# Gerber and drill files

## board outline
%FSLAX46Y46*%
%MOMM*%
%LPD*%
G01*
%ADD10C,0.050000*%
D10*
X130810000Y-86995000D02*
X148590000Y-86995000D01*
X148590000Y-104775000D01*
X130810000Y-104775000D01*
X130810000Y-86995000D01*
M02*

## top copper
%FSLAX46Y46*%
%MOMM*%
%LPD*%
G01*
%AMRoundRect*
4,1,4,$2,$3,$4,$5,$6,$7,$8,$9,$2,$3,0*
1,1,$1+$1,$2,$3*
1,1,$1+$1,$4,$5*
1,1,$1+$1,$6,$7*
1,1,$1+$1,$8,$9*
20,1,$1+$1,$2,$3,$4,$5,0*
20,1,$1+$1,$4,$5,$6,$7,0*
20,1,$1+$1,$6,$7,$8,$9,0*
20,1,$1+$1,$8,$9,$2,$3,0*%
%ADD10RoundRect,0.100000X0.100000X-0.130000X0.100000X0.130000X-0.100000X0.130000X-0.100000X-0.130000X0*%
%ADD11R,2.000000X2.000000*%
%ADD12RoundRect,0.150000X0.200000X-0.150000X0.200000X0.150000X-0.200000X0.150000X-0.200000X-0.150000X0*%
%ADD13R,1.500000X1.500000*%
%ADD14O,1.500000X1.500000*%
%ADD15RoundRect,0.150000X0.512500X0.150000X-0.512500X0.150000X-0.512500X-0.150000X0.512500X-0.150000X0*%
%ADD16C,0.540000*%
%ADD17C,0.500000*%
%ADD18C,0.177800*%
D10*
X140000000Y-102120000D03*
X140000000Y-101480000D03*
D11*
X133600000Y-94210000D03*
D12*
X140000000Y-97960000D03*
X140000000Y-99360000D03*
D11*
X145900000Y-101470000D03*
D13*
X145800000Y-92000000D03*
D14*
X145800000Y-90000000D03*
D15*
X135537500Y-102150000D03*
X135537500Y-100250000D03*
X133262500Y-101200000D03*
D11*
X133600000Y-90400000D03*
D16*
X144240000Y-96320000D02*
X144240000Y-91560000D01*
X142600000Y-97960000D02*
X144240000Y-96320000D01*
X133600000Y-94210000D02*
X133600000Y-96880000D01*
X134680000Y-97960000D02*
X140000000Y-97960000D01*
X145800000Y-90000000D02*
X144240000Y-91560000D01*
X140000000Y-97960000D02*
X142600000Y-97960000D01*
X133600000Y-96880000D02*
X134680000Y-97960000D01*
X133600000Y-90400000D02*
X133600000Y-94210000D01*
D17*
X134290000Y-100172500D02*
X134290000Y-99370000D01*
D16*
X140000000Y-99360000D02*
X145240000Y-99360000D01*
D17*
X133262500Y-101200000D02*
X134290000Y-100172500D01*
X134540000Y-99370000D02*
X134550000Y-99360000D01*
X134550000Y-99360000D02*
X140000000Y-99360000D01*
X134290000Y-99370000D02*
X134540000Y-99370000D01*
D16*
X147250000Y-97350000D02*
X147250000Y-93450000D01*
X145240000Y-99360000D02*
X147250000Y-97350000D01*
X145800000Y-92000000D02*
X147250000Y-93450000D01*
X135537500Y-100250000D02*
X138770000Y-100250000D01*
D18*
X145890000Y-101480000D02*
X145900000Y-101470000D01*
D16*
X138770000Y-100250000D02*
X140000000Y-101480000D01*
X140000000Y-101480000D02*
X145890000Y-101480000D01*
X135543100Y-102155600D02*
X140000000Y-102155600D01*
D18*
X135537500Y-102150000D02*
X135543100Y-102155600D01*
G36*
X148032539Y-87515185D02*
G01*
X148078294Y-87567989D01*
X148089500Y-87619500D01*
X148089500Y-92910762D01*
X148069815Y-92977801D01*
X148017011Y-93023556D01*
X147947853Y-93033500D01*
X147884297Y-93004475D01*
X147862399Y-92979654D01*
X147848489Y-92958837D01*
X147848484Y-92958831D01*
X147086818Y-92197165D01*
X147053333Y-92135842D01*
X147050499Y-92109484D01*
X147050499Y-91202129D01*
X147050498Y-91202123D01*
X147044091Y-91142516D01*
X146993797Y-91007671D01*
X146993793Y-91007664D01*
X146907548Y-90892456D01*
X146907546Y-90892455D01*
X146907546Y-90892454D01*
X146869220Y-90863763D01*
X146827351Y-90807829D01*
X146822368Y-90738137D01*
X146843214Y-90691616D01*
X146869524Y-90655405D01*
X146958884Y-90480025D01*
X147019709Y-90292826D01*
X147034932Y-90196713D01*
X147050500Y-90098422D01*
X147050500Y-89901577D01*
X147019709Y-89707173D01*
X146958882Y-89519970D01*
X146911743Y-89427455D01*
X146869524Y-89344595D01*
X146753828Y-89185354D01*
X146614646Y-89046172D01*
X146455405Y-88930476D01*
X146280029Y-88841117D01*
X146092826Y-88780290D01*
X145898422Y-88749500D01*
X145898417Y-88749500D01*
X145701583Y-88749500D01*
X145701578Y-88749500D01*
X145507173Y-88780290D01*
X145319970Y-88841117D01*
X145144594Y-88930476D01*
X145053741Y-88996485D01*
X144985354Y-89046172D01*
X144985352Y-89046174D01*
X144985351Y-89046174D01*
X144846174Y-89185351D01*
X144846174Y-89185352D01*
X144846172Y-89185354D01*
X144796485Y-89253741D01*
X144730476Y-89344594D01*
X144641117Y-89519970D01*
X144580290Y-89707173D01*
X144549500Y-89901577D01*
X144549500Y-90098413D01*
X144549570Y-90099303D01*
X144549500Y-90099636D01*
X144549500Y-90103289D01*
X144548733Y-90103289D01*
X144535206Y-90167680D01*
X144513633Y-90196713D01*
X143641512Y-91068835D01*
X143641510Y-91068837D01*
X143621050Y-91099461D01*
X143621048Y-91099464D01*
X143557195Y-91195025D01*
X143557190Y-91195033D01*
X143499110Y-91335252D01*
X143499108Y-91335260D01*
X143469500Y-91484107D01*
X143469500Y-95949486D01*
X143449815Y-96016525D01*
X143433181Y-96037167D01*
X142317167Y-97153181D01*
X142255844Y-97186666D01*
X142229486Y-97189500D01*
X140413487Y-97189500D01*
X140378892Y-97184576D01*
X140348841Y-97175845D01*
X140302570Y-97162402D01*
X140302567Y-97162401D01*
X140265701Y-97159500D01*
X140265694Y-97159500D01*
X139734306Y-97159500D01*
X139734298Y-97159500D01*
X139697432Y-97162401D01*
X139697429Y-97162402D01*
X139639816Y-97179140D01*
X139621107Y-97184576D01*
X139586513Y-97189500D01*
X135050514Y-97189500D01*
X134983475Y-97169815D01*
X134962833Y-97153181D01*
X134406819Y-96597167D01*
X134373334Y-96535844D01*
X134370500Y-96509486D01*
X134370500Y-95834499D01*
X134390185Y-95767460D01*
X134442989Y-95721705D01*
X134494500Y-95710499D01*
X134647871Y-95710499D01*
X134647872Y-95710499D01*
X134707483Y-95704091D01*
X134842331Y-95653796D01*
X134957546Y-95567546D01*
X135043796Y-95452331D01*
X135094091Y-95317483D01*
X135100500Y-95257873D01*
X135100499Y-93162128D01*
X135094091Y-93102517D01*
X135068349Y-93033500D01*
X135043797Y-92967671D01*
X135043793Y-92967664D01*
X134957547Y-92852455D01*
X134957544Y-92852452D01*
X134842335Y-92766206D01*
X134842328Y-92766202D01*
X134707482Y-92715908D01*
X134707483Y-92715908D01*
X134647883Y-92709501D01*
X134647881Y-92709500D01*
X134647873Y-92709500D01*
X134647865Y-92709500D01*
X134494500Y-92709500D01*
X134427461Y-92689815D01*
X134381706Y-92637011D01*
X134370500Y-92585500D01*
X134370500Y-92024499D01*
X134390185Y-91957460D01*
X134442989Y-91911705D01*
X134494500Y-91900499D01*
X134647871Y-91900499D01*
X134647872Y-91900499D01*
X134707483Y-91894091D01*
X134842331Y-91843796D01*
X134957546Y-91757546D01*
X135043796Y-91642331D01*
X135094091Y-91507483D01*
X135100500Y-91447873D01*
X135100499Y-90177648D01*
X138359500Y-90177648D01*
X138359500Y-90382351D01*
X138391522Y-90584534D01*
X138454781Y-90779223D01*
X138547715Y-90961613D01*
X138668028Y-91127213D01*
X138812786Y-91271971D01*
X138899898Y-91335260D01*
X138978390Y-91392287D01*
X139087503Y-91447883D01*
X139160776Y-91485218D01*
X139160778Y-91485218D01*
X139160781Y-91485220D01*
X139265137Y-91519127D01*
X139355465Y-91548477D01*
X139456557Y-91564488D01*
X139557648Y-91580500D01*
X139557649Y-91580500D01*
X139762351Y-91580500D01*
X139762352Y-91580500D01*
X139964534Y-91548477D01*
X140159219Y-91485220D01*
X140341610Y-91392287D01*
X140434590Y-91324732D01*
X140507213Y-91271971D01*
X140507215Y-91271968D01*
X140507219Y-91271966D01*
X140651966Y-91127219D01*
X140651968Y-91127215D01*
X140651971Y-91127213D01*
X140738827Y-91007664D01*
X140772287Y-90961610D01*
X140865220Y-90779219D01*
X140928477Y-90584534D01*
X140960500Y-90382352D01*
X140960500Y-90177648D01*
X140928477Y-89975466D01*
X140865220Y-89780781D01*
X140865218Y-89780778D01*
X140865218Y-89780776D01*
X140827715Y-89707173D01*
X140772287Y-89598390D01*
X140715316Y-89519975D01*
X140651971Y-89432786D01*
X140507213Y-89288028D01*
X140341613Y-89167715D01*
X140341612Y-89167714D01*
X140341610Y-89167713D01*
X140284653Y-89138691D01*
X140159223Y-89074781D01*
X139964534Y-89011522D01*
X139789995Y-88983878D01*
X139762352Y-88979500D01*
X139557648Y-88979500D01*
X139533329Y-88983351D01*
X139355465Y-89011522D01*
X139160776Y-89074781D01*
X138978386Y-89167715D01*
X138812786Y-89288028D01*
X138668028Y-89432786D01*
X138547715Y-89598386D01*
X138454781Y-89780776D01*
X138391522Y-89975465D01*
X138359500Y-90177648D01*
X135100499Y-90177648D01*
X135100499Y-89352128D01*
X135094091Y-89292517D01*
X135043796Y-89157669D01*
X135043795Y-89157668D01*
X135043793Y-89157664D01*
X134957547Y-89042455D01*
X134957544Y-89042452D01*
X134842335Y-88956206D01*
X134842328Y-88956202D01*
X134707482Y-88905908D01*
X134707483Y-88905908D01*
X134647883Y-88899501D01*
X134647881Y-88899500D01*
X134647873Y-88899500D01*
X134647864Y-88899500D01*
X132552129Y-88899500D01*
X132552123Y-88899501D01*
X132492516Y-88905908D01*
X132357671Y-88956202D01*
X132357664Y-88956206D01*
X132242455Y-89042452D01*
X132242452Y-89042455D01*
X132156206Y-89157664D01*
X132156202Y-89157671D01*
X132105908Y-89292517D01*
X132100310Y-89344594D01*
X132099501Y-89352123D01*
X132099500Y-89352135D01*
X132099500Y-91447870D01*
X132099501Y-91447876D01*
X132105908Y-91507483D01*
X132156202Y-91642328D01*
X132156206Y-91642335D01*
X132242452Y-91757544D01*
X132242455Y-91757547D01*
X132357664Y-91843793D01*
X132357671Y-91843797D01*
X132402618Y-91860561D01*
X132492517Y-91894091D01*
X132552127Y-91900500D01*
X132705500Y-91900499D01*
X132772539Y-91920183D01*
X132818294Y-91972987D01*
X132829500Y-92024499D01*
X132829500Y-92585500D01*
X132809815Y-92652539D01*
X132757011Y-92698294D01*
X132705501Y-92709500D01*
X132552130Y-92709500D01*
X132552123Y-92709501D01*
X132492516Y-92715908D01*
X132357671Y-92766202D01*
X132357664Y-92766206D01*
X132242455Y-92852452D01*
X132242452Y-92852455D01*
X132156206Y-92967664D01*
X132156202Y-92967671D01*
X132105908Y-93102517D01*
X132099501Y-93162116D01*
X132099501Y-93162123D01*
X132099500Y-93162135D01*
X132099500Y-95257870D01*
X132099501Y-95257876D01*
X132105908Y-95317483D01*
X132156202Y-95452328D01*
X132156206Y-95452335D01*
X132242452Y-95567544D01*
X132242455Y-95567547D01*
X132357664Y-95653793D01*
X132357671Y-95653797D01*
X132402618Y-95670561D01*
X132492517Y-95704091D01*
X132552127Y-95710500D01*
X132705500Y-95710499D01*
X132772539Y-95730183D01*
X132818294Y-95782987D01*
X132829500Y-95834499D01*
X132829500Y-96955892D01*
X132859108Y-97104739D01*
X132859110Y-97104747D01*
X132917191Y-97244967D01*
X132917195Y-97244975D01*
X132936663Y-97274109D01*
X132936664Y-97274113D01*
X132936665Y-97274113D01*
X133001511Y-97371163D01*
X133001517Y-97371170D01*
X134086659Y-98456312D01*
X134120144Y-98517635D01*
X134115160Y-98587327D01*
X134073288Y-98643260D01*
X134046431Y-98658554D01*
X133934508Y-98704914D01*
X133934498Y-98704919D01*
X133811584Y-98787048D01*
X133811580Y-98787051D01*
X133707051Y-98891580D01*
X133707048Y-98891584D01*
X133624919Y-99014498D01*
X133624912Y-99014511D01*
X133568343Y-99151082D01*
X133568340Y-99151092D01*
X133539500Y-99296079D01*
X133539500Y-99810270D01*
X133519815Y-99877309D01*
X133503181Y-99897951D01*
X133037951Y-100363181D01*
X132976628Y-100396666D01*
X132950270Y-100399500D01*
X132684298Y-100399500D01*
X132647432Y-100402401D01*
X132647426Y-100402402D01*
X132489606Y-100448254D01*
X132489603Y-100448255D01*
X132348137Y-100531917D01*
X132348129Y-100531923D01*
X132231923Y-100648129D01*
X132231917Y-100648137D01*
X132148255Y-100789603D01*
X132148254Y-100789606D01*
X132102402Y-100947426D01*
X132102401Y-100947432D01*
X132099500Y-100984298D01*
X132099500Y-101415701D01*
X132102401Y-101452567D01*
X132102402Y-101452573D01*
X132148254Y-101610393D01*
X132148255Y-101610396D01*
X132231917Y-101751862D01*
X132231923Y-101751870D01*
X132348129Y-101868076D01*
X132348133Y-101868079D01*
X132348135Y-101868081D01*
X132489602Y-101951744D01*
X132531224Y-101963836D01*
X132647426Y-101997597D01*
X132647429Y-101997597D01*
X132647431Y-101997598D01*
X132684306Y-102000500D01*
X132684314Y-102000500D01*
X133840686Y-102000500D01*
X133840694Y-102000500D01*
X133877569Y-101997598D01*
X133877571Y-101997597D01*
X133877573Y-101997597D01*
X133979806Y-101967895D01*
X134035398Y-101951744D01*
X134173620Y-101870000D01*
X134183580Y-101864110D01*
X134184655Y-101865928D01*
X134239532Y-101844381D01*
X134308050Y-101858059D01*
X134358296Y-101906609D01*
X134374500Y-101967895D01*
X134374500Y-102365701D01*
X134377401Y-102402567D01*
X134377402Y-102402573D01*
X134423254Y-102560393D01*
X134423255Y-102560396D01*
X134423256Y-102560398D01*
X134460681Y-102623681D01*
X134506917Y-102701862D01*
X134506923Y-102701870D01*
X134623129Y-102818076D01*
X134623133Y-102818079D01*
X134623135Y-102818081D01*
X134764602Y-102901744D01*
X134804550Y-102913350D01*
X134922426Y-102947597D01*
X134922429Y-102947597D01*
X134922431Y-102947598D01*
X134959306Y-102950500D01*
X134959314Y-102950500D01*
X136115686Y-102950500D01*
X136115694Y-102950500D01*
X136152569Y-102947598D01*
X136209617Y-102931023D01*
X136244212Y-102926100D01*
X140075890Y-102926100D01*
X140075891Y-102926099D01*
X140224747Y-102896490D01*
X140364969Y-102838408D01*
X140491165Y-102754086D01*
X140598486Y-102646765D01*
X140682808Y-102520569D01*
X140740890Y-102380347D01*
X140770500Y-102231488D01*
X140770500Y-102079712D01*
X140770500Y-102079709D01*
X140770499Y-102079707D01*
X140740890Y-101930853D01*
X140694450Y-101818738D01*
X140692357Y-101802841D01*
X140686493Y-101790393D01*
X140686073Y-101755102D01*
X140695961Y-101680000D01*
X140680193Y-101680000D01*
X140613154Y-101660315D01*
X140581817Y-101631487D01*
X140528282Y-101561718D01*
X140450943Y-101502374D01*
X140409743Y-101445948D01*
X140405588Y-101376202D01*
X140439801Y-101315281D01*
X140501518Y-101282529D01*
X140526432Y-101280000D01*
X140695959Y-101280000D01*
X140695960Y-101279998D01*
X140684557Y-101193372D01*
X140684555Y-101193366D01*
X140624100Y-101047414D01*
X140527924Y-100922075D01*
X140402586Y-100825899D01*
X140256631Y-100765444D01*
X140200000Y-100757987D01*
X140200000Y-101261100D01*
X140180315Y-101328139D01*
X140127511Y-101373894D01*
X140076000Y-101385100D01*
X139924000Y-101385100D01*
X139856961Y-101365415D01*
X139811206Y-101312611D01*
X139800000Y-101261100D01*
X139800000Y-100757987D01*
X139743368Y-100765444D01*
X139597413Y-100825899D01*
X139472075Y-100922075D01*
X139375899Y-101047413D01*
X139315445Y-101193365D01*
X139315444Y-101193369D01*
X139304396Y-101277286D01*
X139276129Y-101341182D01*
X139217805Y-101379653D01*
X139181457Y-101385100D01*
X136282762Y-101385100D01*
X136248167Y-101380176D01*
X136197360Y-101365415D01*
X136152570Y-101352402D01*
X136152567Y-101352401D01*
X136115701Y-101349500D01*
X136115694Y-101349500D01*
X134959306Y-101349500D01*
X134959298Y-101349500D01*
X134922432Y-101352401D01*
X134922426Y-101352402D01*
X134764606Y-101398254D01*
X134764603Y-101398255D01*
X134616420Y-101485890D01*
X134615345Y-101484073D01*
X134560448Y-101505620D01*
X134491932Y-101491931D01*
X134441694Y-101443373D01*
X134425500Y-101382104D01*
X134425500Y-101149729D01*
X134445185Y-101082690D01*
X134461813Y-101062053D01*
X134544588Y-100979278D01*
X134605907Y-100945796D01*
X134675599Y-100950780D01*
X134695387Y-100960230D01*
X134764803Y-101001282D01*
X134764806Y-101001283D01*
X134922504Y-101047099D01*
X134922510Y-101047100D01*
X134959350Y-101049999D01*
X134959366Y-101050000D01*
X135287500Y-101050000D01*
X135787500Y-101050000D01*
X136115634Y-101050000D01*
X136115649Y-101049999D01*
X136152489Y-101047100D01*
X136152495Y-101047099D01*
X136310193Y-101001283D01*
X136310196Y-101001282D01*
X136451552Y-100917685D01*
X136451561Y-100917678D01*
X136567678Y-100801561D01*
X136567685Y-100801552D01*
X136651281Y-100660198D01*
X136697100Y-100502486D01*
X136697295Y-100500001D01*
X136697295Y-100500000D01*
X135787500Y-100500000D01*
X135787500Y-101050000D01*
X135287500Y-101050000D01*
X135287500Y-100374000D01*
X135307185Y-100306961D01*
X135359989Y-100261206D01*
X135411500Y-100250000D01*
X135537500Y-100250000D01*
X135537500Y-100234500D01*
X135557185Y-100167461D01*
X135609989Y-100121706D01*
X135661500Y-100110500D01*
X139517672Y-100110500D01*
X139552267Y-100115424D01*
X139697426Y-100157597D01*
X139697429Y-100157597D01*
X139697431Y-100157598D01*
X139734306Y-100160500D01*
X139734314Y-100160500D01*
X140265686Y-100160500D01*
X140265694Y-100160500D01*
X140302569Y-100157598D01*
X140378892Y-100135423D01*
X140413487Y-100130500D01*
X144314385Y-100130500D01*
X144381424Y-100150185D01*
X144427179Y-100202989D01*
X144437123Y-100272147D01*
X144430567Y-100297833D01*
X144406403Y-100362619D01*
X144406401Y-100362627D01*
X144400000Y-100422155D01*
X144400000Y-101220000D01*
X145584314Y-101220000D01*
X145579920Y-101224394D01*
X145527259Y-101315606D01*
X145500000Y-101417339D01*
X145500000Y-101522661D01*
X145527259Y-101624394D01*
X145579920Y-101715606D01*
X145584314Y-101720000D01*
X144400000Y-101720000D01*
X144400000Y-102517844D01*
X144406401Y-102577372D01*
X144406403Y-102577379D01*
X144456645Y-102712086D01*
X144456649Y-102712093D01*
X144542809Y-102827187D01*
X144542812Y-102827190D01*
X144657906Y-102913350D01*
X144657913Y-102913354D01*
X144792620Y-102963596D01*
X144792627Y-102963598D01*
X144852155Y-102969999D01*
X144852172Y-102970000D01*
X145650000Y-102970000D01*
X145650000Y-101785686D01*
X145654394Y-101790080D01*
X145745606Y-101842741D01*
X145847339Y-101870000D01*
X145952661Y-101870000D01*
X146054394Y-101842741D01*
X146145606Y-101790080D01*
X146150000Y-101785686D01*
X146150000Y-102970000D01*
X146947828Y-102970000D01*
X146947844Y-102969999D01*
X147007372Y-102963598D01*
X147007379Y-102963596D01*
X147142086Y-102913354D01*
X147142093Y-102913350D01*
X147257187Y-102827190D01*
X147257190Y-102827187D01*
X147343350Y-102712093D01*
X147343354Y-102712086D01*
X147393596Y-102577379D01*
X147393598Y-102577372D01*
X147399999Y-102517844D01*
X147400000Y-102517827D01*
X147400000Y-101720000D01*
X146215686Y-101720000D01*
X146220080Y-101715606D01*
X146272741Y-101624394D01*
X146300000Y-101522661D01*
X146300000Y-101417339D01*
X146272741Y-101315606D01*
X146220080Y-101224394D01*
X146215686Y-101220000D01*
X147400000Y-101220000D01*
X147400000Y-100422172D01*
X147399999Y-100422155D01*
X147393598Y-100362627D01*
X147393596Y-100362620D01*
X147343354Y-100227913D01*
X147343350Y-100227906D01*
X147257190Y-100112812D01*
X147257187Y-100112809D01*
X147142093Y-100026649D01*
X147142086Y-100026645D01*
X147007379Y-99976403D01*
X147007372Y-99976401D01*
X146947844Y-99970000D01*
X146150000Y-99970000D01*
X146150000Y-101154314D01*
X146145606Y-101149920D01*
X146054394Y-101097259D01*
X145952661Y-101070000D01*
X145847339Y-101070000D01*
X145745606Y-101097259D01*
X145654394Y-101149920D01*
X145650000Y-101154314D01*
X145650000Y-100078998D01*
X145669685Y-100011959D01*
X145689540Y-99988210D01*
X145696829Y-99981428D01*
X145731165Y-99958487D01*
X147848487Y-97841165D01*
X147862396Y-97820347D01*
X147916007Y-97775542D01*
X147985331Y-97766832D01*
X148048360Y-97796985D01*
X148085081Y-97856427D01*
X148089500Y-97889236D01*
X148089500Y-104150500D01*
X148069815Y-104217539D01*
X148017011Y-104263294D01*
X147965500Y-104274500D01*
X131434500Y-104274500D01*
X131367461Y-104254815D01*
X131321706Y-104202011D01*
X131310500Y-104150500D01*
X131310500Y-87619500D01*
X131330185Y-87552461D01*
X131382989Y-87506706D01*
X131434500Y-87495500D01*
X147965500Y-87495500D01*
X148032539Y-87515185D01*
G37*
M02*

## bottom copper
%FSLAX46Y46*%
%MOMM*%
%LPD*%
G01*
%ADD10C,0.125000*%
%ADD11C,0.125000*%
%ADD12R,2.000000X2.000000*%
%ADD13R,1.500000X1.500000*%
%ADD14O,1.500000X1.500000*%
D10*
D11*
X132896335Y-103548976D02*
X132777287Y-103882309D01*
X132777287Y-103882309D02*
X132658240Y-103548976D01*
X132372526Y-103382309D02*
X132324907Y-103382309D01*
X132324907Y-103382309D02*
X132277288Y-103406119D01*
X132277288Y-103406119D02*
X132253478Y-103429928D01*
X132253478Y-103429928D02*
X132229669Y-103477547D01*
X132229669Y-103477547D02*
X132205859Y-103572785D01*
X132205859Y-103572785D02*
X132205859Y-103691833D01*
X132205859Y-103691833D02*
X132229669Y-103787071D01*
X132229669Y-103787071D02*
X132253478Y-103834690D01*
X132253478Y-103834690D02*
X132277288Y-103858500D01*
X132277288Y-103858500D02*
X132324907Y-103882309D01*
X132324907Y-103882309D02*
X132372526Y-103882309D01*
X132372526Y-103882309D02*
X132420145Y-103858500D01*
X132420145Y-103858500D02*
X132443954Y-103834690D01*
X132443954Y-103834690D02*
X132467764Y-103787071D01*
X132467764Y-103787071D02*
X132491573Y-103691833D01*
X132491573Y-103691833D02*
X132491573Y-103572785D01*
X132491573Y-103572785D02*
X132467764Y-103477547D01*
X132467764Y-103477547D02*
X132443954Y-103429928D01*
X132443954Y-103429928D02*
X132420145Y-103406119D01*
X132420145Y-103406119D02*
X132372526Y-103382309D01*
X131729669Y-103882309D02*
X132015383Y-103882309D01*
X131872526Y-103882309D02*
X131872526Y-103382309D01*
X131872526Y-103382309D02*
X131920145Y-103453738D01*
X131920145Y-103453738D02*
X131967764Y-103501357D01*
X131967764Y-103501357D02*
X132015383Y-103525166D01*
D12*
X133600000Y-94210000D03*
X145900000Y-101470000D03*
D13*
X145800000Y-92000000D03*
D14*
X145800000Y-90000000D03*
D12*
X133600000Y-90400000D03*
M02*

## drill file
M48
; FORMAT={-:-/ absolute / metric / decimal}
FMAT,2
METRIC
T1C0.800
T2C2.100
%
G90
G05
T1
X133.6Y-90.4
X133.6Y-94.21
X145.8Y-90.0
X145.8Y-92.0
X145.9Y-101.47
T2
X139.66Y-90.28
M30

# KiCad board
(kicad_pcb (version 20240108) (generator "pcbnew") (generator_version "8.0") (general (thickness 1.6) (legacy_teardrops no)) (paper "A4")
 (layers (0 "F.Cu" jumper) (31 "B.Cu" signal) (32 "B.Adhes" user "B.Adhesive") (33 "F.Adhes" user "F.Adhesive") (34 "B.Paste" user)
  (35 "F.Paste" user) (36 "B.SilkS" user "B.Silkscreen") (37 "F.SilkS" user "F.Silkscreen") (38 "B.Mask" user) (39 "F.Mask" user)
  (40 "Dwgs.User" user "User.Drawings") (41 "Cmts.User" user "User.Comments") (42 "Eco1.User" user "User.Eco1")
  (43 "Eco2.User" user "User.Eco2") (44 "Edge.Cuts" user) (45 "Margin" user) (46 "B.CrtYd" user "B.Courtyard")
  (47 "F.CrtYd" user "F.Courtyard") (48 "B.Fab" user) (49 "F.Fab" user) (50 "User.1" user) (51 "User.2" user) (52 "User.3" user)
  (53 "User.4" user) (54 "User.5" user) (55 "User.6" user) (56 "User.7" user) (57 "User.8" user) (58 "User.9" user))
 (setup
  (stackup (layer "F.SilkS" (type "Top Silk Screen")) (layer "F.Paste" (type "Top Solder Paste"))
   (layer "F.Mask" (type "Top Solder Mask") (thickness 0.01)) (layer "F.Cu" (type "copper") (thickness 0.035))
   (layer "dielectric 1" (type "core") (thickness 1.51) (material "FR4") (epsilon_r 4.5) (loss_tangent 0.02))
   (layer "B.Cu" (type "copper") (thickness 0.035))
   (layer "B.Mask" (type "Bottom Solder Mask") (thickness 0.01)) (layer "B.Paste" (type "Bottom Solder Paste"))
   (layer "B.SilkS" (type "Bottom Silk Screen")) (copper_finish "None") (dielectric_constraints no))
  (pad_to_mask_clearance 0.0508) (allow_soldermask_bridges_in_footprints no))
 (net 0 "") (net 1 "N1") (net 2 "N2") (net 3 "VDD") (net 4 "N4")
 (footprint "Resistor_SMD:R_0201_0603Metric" (layer "F.Cu") (at 140 101.8 90)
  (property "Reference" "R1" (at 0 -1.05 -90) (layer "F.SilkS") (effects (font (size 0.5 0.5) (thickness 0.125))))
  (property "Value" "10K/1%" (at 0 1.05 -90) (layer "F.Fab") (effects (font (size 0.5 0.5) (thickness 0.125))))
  (pad "" smd roundrect (at -0.345 0 90) (size 0.318 0.36) (layers "F.Paste") (roundrect_rratio 0.25))
  (pad "" smd roundrect (at 0.345 0 90) (size 0.318 0.36) (layers "F.Paste") (roundrect_rratio 0.25))
  (pad "1" smd roundrect (at -0.32 0 90) (size 0.46 0.4) (layers "F.Cu" "F.Mask") (roundrect_rratio 0.25) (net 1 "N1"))
  (pad "2" smd roundrect (at 0.32 0 90) (size 0.46 0.4) (layers "F.Cu" "F.Mask") (roundrect_rratio 0.25) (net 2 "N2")))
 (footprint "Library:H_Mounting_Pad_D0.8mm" (layer "F.Cu") (at 133.6 94.21)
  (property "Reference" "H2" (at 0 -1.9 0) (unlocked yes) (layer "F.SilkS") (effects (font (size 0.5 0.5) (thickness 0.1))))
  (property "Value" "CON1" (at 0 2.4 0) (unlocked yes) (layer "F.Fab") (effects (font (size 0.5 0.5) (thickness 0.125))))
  (pad "1" thru_hole rect (at 0 0) (size 2 2) (drill 0.8) (layers "*.Cu" "*.Mask") (remove_unused_layers no) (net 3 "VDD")))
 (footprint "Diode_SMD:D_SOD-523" (layer "F.Cu") (at 140 98.66 -90)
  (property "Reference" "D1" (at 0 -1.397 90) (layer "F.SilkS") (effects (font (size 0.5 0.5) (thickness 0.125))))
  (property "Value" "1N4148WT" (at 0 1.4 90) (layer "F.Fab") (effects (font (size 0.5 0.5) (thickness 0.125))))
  (pad "1" smd roundrect (at -0.7 0 90) (size 0.6 0.7) (layers "F.Cu" "F.Paste" "F.Mask") (roundrect_rratio 0.25) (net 3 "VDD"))
  (pad "2" smd roundrect (at 0.7 0 90) (size 0.6 0.7) (layers "F.Cu" "F.Paste" "F.Mask") (roundrect_rratio 0.25) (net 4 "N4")))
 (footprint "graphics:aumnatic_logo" (layer "F.Cu") (at 140.95 96)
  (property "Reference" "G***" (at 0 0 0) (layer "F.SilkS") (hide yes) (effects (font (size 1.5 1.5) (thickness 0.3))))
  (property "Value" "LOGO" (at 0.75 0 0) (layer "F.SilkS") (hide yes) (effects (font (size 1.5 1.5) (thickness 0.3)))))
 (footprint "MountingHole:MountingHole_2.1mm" (layer "F.Cu") (at 139.66 90.28)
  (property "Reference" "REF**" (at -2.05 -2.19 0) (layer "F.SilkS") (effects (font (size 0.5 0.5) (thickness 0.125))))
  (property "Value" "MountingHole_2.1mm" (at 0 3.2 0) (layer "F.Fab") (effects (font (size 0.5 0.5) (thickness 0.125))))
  (pad "" np_thru_hole circle (at 0 0) (size 2.1 2.1) (drill 2.1) (layers "*.Cu" "*.Mask")))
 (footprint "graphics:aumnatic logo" (layer "F.Cu") (at 139.6 94.65)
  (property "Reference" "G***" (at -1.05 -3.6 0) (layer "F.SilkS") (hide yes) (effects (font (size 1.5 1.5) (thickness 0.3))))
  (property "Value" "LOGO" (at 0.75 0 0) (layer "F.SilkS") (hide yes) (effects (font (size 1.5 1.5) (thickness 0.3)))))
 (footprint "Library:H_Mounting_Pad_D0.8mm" (layer "F.Cu") (at 145.9 101.47)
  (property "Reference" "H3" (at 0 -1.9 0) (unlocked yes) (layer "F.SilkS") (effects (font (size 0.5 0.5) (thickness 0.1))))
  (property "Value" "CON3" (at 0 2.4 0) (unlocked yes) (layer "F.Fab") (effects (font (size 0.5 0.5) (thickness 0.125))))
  (pad "1" thru_hole rect (at 0 0) (size 2 2) (drill 0.8) (layers "*.Cu" "*.Mask") (remove_unused_layers no) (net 2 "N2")))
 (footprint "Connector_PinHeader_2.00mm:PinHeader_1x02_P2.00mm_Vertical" (layer "F.Cu") (at 145.8 92 180)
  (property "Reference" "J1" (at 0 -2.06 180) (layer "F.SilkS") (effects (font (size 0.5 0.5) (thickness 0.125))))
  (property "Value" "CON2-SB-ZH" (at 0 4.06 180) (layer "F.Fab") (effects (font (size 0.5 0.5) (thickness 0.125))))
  (pad "1" thru_hole rect (at 0 0 180) (size 1.5 1.5) (drill 0.8) (layers "*.Cu" "*.Mask") (remove_unused_layers no) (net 4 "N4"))
  (pad "2" thru_hole oval (at 0 2 180) (size 1.5 1.5) (drill 0.8) (layers "*.Cu" "*.Mask") (remove_unused_layers no) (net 3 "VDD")))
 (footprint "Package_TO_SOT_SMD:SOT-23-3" (layer "F.Cu") (at 134.4 101.2 180)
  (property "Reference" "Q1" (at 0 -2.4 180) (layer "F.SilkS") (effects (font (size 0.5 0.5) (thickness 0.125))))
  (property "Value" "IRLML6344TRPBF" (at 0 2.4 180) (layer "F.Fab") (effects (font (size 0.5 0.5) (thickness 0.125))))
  (pad "1" smd roundrect (at -1.1375 -0.95 180) (size 1.325 0.6) (layers "F.Cu" "F.Paste" "F.Mask") (roundrect_rratio 0.25) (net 1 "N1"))
  (pad "2" smd roundrect (at -1.1375 0.95 180) (size 1.325 0.6) (layers "F.Cu" "F.Paste" "F.Mask") (roundrect_rratio 0.25) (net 2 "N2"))
  (pad "3" smd roundrect (at 1.1375 0 180) (size 1.325 0.6) (layers "F.Cu" "F.Paste" "F.Mask") (roundrect_rratio 0.25) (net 4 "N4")))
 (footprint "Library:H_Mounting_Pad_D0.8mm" (layer "F.Cu") (at 133.6 90.4)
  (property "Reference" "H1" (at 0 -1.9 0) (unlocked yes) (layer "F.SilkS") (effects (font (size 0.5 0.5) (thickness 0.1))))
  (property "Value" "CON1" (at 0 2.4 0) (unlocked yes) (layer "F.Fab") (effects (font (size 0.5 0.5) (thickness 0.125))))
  (pad "1" thru_hole rect (at 0 0) (size 2 2) (drill 0.8) (layers "*.Cu" "*.Mask") (remove_unused_layers no) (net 3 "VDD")))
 (gr_rect (start 130.81 86.995) (end 148.59 104.775) (stroke (width 0.05) (type default)) (fill none) (layer "Edge.Cuts"))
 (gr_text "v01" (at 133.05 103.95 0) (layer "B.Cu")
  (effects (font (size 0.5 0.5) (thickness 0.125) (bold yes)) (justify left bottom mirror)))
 (segment (start 144.24 96.32) (end 144.24 91.56) (width 0.54) (layer "F.Cu") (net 3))
 (segment (start 142.6 97.96) (end 144.24 96.32) (width 0.54) (layer "F.Cu") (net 3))
 (segment (start 133.6 94.21) (end 133.6 96.88) (width 0.54) (layer "F.Cu") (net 3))
 (segment (start 134.68 97.96) (end 140 97.96) (width 0.54) (layer "F.Cu") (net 3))
 (segment (start 145.8 90) (end 144.24 91.56) (width 0.54) (layer "F.Cu") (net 3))
 (segment (start 140 97.96) (end 142.6 97.96) (width 0.54) (layer "F.Cu") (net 3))
 (segment (start 133.6 96.88) (end 134.68 97.96) (width 0.54) (layer "F.Cu") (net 3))
 (segment (start 133.6 90.4) (end 133.6 94.21) (width 0.54) (layer "F.Cu") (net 3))
 (segment (start 134.29 100.1725) (end 134.29 99.37) (width 0.5) (layer "F.Cu") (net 4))
 (segment (start 140 99.36) (end 145.24 99.36) (width 0.54) (layer "F.Cu") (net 4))
 (segment (start 133.2625 101.2) (end 134.29 100.1725) (width 0.5) (layer "F.Cu") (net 4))
 (segment (start 134.54 99.37) (end 134.55 99.36) (width 0.5) (layer "F.Cu") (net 4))
 (segment (start 134.55 99.36) (end 140 99.36) (width 0.5) (layer "F.Cu") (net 4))
 (segment (start 134.29 99.37) (end 134.54 99.37) (width 0.5) (layer "F.Cu") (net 4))
 (segment (start 147.25 97.35) (end 147.25 93.45) (width 0.54) (layer "F.Cu") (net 4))
 (segment (start 145.24 99.36) (end 147.25 97.35) (width 0.54) (layer "F.Cu") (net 4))
 (segment (start 145.8 92) (end 147.25 93.45) (width 0.54) (layer "F.Cu") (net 4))
 (segment (start 135.5375 100.25) (end 138.77 100.25) (width 0.54) (layer "F.Cu") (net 2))
 (segment (start 145.89 101.48) (end 145.9 101.47) (width 0.1778) (layer "F.Cu") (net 2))
 (segment (start 138.77 100.25) (end 140 101.48) (width 0.54) (layer "F.Cu") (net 2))
 (segment (start 140 101.48) (end 145.89 101.48) (width 0.54) (layer "F.Cu") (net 2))
 (segment (start 135.5431 102.1556) (end 140 102.1556) (width 0.54) (layer "F.Cu") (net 1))
 (segment (start 135.5375 102.15) (end 135.5431 102.1556) (width 0.1778) (layer "F.Cu") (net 1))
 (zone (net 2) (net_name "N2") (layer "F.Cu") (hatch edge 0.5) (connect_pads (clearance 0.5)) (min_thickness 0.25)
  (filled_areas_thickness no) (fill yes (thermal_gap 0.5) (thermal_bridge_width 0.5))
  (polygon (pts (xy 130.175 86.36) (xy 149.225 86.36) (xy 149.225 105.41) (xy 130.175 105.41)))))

